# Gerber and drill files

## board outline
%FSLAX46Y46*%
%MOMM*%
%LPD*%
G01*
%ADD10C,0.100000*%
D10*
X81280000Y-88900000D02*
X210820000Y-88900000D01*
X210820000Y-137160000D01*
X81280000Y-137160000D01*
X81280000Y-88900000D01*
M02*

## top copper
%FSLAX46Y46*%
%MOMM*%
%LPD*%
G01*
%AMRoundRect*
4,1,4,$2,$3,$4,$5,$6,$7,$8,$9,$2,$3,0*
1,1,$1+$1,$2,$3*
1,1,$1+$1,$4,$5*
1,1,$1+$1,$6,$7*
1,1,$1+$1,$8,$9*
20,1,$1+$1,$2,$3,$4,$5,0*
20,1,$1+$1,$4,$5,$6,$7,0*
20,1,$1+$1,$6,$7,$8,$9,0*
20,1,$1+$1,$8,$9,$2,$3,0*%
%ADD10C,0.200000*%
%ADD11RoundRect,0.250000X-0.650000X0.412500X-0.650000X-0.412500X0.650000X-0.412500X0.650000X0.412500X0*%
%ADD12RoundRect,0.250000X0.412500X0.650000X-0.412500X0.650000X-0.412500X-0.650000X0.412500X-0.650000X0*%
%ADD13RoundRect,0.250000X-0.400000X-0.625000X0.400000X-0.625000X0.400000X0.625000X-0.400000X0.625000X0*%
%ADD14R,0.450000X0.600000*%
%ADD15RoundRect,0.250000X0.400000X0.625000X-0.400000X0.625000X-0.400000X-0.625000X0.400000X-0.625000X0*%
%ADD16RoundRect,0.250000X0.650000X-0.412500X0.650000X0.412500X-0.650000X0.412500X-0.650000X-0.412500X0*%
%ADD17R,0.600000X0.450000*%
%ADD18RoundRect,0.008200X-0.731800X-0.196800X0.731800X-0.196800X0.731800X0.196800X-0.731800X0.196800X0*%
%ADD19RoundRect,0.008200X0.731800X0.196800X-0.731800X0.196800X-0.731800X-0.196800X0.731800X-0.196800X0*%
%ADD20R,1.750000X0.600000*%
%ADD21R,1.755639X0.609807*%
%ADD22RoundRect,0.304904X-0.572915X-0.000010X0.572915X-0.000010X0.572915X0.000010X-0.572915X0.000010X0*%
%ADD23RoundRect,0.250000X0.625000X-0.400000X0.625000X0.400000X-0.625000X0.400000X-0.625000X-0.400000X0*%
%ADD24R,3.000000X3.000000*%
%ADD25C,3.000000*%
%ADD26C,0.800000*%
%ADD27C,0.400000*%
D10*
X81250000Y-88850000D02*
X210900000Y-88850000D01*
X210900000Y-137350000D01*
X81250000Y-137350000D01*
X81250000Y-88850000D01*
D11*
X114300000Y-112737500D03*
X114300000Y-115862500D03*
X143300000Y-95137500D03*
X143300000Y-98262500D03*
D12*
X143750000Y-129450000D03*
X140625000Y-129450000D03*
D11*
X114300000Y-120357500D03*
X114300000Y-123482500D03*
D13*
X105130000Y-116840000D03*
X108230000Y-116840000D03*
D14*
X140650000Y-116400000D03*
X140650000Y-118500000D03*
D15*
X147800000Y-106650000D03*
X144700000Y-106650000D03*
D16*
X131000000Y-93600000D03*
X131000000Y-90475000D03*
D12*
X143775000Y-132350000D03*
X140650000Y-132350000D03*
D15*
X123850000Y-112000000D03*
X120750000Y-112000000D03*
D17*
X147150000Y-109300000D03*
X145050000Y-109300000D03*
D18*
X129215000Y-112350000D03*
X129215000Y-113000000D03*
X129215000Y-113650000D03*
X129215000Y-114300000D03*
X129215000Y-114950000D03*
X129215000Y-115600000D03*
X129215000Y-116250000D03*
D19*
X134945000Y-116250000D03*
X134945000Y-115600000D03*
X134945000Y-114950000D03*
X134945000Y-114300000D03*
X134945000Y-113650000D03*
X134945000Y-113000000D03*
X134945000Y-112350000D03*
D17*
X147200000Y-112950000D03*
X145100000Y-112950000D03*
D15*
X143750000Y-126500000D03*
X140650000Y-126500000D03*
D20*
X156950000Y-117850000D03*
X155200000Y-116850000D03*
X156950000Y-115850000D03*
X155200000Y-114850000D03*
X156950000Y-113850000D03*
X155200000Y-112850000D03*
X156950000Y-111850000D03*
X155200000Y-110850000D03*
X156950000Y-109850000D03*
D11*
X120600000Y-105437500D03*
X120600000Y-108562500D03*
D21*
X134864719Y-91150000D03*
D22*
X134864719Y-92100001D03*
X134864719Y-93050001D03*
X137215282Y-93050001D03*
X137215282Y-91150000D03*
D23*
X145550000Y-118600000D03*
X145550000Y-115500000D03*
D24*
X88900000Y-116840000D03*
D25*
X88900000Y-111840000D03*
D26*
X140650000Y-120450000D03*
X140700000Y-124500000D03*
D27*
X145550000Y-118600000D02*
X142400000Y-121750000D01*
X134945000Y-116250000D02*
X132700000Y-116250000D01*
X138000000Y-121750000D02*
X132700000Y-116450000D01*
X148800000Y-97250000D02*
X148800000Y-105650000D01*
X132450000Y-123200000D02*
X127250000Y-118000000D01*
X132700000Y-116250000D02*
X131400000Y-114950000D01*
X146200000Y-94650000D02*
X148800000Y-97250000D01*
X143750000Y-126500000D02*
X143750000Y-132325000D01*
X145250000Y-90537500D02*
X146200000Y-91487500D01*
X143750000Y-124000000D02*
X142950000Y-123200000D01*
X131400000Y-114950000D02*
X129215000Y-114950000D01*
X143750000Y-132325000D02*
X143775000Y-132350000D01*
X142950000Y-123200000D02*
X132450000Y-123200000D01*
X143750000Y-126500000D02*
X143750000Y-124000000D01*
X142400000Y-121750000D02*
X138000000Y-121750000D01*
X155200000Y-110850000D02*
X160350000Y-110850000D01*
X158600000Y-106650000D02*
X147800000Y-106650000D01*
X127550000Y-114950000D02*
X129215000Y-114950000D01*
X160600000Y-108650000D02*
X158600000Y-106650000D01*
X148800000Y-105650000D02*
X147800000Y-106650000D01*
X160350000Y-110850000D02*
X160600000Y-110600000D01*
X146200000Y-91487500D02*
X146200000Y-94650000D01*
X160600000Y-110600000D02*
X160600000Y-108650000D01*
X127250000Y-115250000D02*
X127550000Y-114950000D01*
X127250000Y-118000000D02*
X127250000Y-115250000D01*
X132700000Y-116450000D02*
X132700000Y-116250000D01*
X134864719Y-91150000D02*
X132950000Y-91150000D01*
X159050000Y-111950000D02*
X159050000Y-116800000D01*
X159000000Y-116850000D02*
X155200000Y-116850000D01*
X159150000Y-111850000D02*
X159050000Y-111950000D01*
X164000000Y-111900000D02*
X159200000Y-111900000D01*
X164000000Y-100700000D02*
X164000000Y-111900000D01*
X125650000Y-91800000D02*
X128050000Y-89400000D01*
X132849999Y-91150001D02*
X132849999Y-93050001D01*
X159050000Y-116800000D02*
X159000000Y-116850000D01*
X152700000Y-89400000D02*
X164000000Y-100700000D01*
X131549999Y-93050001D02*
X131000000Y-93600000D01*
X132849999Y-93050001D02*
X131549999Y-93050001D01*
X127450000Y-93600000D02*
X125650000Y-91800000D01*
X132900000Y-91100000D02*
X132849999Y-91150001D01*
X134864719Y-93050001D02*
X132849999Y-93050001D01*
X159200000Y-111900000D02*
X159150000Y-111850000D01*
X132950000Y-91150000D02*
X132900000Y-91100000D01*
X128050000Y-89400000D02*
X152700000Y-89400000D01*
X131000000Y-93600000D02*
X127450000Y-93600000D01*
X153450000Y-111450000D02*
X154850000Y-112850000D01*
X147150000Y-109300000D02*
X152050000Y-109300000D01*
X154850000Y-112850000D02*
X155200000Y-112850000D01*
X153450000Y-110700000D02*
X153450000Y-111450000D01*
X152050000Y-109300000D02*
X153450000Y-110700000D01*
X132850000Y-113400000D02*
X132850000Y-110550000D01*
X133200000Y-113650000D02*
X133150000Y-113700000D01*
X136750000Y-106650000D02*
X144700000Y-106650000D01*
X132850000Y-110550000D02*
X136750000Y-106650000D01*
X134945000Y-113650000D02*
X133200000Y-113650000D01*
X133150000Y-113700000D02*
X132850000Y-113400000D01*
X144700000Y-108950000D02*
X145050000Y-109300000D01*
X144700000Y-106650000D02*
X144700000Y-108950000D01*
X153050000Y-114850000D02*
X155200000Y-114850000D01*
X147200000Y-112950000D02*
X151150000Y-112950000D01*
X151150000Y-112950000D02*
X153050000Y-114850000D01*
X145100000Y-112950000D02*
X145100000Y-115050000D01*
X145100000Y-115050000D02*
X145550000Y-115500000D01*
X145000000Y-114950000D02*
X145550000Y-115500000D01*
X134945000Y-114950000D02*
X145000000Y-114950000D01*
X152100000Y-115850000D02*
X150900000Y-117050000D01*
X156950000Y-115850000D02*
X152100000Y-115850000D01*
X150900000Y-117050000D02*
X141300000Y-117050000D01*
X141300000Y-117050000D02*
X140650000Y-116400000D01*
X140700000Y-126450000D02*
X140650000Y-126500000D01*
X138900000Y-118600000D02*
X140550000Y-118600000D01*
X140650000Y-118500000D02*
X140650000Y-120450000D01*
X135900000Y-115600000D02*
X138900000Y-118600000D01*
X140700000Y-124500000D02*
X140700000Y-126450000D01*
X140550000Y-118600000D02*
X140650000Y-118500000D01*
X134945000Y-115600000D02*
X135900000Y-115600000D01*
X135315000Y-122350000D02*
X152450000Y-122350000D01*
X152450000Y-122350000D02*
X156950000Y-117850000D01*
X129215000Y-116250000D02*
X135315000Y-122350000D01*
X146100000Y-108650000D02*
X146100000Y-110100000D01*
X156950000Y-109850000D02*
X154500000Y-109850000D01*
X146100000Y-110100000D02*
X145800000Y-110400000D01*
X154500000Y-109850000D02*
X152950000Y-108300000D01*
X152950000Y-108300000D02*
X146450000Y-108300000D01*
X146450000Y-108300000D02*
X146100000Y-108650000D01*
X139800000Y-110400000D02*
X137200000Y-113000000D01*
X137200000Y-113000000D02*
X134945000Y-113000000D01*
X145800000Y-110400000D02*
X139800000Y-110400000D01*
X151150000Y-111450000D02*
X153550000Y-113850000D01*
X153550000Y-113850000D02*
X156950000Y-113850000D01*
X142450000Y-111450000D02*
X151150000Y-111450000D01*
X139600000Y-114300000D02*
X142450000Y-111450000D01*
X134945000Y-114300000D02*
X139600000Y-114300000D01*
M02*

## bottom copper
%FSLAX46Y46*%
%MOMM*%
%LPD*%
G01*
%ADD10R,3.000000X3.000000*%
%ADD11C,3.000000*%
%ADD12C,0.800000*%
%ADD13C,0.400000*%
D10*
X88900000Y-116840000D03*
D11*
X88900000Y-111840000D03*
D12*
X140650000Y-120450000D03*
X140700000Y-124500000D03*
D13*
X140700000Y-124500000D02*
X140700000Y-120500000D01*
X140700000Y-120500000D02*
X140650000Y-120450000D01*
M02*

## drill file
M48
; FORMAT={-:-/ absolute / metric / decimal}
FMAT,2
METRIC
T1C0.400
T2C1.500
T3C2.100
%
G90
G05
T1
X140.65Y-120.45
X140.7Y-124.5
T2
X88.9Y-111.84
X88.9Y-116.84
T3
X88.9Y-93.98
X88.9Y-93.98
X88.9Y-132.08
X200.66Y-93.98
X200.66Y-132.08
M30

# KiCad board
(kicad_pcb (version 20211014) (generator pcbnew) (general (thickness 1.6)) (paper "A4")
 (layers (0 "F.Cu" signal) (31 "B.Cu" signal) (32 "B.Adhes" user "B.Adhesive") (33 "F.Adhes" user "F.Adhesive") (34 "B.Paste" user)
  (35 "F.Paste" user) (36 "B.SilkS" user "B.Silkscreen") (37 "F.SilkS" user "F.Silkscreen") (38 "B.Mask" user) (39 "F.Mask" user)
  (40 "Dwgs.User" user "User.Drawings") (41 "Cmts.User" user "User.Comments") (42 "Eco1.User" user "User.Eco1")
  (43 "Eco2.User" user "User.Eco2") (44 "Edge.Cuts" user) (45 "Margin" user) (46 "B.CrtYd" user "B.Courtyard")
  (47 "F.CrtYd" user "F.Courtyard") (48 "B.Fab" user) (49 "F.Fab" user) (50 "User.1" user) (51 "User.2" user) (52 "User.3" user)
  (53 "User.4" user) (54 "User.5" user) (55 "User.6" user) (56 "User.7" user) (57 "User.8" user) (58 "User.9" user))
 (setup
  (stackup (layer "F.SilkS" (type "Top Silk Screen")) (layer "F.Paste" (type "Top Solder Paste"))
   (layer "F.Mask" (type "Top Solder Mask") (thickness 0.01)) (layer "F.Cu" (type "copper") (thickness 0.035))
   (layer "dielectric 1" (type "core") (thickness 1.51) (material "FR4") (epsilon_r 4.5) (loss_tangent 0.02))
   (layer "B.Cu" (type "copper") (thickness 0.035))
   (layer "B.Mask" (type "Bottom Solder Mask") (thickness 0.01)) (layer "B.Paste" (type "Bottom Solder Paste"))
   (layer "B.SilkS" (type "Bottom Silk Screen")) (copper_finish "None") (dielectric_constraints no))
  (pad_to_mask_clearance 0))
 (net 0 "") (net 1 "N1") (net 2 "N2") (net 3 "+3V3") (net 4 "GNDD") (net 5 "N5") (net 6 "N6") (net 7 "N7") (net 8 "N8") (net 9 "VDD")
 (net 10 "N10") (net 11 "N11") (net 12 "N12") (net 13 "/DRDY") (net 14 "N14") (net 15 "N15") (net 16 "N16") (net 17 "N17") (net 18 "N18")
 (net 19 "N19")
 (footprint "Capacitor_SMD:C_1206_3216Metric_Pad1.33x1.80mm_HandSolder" (layer "F.Cu") (at 114.3 114.3 -90)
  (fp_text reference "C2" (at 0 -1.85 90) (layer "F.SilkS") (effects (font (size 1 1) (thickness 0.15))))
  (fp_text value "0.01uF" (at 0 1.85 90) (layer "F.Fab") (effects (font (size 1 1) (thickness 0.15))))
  (pad "1" smd roundrect (at -1.5625 0 270) (size 1.325 1.8) (layers "F.Cu" "F.Paste" "F.Mask") (roundrect_rratio 0.188679) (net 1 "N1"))
  (pad "2" smd roundrect (at 1.5625 0 270) (size 1.325 1.8) (layers "F.Cu" "F.Paste" "F.Mask") (roundrect_rratio 0.188679) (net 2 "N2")))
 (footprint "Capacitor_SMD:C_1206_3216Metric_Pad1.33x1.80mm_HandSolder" (layer "F.Cu") (at 143.3 96.7 -90)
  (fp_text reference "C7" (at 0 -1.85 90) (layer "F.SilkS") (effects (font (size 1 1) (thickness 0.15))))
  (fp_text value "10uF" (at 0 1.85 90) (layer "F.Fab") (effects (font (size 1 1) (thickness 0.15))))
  (pad "1" smd roundrect (at -1.5625 0 270) (size 1.325 1.8) (layers "F.Cu" "F.Paste" "F.Mask") (roundrect_rratio 0.188679) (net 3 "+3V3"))
  (pad "2" smd roundrect (at 1.5625 0 270) (size 1.325 1.8) (layers "F.Cu" "F.Paste" "F.Mask") (roundrect_rratio 0.188679) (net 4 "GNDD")))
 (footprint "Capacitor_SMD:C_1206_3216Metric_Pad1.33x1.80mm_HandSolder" (layer "F.Cu") (at 142.1875 129.45 180)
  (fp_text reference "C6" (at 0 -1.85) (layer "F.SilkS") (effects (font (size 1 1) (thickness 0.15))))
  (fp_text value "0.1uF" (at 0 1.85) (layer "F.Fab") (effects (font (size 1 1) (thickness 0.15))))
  (pad "1" smd roundrect (at -1.5625 0 180) (size 1.325 1.8) (layers "F.Cu" "F.Paste" "F.Mask") (roundrect_rratio 0.188679) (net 3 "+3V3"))
  (pad "2" smd roundrect (at 1.5625 0 180) (size 1.325 1.8) (layers "F.Cu" "F.Paste" "F.Mask") (roundrect_rratio 0.188679) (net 4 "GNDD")))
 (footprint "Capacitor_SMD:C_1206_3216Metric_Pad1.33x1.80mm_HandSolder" (layer "F.Cu") (at 114.3 121.92 -90)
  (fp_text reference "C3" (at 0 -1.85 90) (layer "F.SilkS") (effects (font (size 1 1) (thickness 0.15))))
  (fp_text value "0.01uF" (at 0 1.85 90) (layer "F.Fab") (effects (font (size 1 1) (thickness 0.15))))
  (pad "1" smd roundrect (at -1.5625 0 270) (size 1.325 1.8) (layers "F.Cu" "F.Paste" "F.Mask") (roundrect_rratio 0.188679) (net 2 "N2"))
  (pad "2" smd roundrect (at 1.5625 0 270) (size 1.325 1.8) (layers "F.Cu" "F.Paste" "F.Mask") (roundrect_rratio 0.188679) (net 4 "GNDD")))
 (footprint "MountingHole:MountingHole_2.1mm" (layer "F.Cu") (at 200.66 132.08)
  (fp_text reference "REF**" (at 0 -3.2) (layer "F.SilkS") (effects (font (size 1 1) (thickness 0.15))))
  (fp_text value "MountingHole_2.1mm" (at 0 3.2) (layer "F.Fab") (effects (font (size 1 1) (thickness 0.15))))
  (pad "" np_thru_hole circle (at 0 0) (size 2.1 2.1) (drill 2.1) (layers *.Cu *.Mask)))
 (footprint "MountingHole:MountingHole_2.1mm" (layer "F.Cu") (at 88.9 93.98)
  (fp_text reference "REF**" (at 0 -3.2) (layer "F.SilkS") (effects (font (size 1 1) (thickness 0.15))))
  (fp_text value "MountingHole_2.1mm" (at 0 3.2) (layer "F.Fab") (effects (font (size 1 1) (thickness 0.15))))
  (pad "" np_thru_hole circle (at 0 0) (size 2.1 2.1) (drill 2.1) (layers *.Cu *.Mask))
  (pad "" np_thru_hole circle (at 0 0) (size 2.1 2.1) (drill 2.1) (layers *.Cu *.Mask)))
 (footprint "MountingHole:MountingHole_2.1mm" (layer "F.Cu") (at 88.9 132.08)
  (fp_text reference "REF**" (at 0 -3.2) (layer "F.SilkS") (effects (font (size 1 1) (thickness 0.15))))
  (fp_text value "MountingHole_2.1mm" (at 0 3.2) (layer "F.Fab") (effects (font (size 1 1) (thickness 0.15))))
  (pad "" np_thru_hole circle (at 0 0) (size 2.1 2.1) (drill 2.1) (layers *.Cu *.Mask)))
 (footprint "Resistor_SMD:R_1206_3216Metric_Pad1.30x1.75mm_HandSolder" (layer "F.Cu") (at 106.68 116.84)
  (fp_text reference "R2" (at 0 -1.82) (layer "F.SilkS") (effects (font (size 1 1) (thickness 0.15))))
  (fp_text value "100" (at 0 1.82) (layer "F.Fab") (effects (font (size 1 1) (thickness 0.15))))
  (pad "1" smd roundrect (at -1.55 0) (size 1.3 1.75) (layers "F.Cu" "F.Paste" "F.Mask") (roundrect_rratio 0.192308) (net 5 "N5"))
  (pad "2" smd roundrect (at 1.55 0) (size 1.3 1.75) (layers "F.Cu" "F.Paste" "F.Mask") (roundrect_rratio 0.192308) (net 2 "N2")))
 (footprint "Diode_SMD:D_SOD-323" (layer "F.Cu") (at 140.65 117.45 -90)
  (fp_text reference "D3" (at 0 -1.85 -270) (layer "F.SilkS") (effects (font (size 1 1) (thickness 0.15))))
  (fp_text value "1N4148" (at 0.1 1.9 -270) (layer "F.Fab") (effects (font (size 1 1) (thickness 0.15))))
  (pad "1" smd rect (at -1.05 0 270) (size 0.6 0.45) (layers "F.Cu" "F.Paste" "F.Mask") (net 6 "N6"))
  (pad "2" smd rect (at 1.05 0 270) (size 0.6 0.45) (layers "F.Cu" "F.Paste" "F.Mask") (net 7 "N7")))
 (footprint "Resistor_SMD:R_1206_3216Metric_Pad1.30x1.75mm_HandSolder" (layer "F.Cu") (at 146.25 106.65 180)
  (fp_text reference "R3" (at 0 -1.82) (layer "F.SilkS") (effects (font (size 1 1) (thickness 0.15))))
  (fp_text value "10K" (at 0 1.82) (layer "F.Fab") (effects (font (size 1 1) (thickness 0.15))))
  (pad "1" smd roundrect (at -1.55 0 180) (size 1.3 1.75) (layers "F.Cu" "F.Paste" "F.Mask") (roundrect_rratio 0.192308) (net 3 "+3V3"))
  (pad "2" smd roundrect (at 1.55 0 180) (size 1.3 1.75) (layers "F.Cu" "F.Paste" "F.Mask") (roundrect_rratio 0.192308) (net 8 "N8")))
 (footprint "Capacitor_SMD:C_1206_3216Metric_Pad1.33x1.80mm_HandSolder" (layer "F.Cu") (at 131 92.0375 90)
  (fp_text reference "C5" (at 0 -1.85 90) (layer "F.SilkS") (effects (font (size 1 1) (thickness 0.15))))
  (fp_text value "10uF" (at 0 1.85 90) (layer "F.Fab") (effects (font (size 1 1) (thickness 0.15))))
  (pad "1" smd roundrect (at -1.5625 0 90) (size 1.325 1.8) (layers "F.Cu" "F.Paste" "F.Mask") (roundrect_rratio 0.188679) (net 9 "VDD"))
  (pad "2" smd roundrect (at 1.5625 0 90) (size 1.325 1.8) (layers "F.Cu" "F.Paste" "F.Mask") (roundrect_rratio 0.188679) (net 4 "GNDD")))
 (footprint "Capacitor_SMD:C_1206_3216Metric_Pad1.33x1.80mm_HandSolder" (layer "F.Cu") (at 142.2125 132.35 180)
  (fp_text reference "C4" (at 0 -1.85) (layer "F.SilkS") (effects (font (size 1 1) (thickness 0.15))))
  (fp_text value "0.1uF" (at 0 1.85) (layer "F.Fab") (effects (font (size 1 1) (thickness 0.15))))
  (pad "1" smd roundrect (at -1.5625 0 180) (size 1.325 1.8) (layers "F.Cu" "F.Paste" "F.Mask") (roundrect_rratio 0.188679) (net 3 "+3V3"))
  (pad "2" smd roundrect (at 1.5625 0 180) (size 1.325 1.8) (layers "F.Cu" "F.Paste" "F.Mask") (roundrect_rratio 0.188679) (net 4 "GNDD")))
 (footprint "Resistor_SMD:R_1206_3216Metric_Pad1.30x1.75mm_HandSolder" (layer "F.Cu") (at 122.3 112 180)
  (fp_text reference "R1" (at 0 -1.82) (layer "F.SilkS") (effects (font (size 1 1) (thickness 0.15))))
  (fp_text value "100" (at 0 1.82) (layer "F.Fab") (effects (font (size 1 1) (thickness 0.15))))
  (pad "1" smd roundrect (at -1.55 0 180) (size 1.3 1.75) (layers "F.Cu" "F.Paste" "F.Mask") (roundrect_rratio 0.192308) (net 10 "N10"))
  (pad "2" smd roundrect (at 1.55 0 180) (size 1.3 1.75) (layers "F.Cu" "F.Paste" "F.Mask") (roundrect_rratio 0.192308) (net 1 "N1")))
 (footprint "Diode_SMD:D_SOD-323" (layer "F.Cu") (at 146.1 109.3 180)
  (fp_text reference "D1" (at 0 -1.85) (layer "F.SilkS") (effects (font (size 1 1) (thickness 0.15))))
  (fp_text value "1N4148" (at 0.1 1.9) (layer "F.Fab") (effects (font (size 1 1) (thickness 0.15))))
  (pad "1" smd rect (at -1.05 0 180) (size 0.6 0.45) (layers "F.Cu" "F.Paste" "F.Mask") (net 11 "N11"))
  (pad "2" smd rect (at 1.05 0 180) (size 0.6 0.45) (layers "F.Cu" "F.Paste" "F.Mask") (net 8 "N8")))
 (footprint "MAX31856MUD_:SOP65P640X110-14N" (layer "F.Cu") (at 132.08 114.3)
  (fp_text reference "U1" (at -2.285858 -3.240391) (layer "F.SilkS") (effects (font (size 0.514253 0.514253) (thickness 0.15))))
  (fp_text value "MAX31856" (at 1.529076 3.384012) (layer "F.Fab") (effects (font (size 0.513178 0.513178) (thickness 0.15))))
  (pad "1" smd roundrect locked (at -2.865 -1.95) (size 1.48 0.41) (layers "F.Cu" "F.Paste" "F.Mask") (roundrect_rratio 0.02) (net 4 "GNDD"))
  (pad "2" smd roundrect locked (at -2.865 -1.3) (size 1.48 0.41) (layers "F.Cu" "F.Paste" "F.Mask") (roundrect_rratio 0.02) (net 10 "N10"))
  (pad "3" smd roundrect locked (at -2.865 -0.65) (size 1.48 0.41) (layers "F.Cu" "F.Paste" "F.Mask") (roundrect_rratio 0.02) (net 1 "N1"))
  (pad "4" smd roundrect locked (at -2.865 0) (size 1.48 0.41) (layers "F.Cu" "F.Paste") (roundrect_rratio 0.02) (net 2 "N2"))
  (pad "5" smd roundrect locked (at -2.865 0.65) (size 1.48 0.41) (layers "F.Cu" "F.Paste" "F.Mask") (roundrect_rratio 0.02) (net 3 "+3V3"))
  (pad "6" smd roundrect locked (at -2.865 1.3) (size 1.48 0.41) (layers "F.Cu" "F.Paste" "F.Mask") (roundrect_rratio 0.02) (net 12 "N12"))
  (pad "7" smd roundrect locked (at -2.865 1.95) (size 1.48 0.41) (layers "F.Cu" "F.Paste" "F.Mask") (roundrect_rratio 0.02)
   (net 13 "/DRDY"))
  (pad "8" smd roundrect locked (at 2.865 1.95 180) (size 1.48 0.41) (layers "F.Cu" "F.Paste" "F.Mask") (roundrect_rratio 0.02)
   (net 3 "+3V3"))
  (pad "9" smd roundrect locked (at 2.865 1.3 180) (size 1.48 0.41) (layers "F.Cu" "F.Paste" "F.Mask") (roundrect_rratio 0.02) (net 7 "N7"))
  (pad "10" smd roundrect locked (at 2.865 0.65 180) (size 1.48 0.41) (layers "F.Cu" "F.Paste" "F.Mask") (roundrect_rratio 0.02)
   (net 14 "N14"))
  (pad "11" smd roundrect locked (at 2.865 0 180) (size 1.48 0.41) (layers "F.Cu" "F.Paste" "F.Mask") (roundrect_rratio 0.02) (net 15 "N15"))
  (pad "12" smd roundrect locked (at 2.865 -0.65 180) (size 1.48 0.41) (layers "F.Cu" "F.Paste" "F.Mask") (roundrect_rratio 0.02)
   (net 8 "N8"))
  (pad "13" smd roundrect locked (at 2.865 -1.3 180) (size 1.48 0.41) (layers "F.Cu" "F.Paste" "F.Mask") (roundrect_rratio 0.02)
   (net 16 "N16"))
  (pad "14" smd roundrect locked (at 2.865 -1.95 180) (size 1.48 0.41) (layers "F.Cu" "F.Paste" "F.Mask") (roundrect_rratio 0.02)
   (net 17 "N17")))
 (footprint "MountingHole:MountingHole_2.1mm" (layer "F.Cu") (at 200.66 93.98)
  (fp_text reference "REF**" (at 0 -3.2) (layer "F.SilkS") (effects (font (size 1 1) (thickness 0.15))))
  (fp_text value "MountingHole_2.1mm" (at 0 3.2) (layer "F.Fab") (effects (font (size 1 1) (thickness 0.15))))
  (pad "" np_thru_hole circle (at 0 0) (size 2.1 2.1) (drill 2.1) (layers *.Cu *.Mask)))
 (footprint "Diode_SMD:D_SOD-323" (layer "F.Cu") (at 146.15 112.95 180)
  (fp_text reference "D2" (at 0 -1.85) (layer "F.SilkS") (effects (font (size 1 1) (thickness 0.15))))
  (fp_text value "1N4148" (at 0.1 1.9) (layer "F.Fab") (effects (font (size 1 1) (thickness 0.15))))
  (pad "1" smd rect (at -1.05 0 180) (size 0.6 0.45) (layers "F.Cu" "F.Paste" "F.Mask") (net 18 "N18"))
  (pad "2" smd rect (at 1.05 0 180) (size 0.6 0.45) (layers "F.Cu" "F.Paste" "F.Mask") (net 14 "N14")))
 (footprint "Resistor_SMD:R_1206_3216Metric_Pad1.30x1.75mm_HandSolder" (layer "F.Cu") (at 142.2 126.5 180)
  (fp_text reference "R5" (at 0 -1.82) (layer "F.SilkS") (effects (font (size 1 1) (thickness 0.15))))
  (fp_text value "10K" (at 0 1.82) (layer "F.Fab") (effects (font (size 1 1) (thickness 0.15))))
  (pad "1" smd roundrect (at -1.55 0 180) (size 1.3 1.75) (layers "F.Cu" "F.Paste" "F.Mask") (roundrect_rratio 0.192308) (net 3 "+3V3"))
  (pad "2" smd roundrect (at 1.55 0 180) (size 1.3 1.75) (layers "F.Cu" "F.Paste" "F.Mask") (roundrect_rratio 0.192308) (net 7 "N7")))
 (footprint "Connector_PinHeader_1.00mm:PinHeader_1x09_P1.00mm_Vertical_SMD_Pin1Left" (layer "F.Cu") (at 156.075 113.85 180)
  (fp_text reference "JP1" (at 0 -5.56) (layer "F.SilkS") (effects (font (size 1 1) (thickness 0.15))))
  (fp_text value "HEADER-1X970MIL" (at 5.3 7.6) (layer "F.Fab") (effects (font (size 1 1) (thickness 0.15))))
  (pad "1" smd rect (at -0.875 -4 180) (size 1.75 0.6) (layers "F.Cu" "F.Paste" "F.Mask") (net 13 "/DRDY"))
  (pad "2" smd rect (at 0.875 -3 180) (size 1.75 0.6) (layers "F.Cu" "F.Paste" "F.Mask") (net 9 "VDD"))
  (pad "3" smd rect (at -0.875 -2 180) (size 1.75 0.6) (layers "F.Cu" "F.Paste" "F.Mask") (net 6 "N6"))
  (pad "4" smd rect (at 0.875 -1 180) (size 1.75 0.6) (layers "F.Cu" "F.Paste" "F.Mask") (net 18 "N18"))
  (pad "5" smd rect (at -0.875 0 180) (size 1.75 0.6) (layers "F.Cu" "F.Paste" "F.Mask") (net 15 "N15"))
  (pad "6" smd rect (at 0.875 1 180) (size 1.75 0.6) (layers "F.Cu" "F.Paste" "F.Mask") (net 11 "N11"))
  (pad "7" smd rect (at -0.875 2 180) (size 1.75 0.6) (layers "F.Cu" "F.Paste" "F.Mask") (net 4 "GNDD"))
  (pad "8" smd rect (at 0.875 3 180) (size 1.75 0.6) (layers "F.Cu" "F.Paste" "F.Mask") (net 3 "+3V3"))
  (pad "9" smd rect (at -0.875 4 180) (size 1.75 0.6) (layers "F.Cu" "F.Paste" "F.Mask") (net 16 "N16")))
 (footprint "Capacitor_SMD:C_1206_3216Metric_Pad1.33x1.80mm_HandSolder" (layer "F.Cu") (at 120.6 107 -90)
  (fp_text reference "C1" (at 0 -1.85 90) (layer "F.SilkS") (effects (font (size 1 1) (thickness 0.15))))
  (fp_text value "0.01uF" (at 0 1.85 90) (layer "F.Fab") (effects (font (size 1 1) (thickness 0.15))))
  (pad "1" smd roundrect (at -1.5625 0 270) (size 1.325 1.8) (layers "F.Cu" "F.Paste" "F.Mask") (roundrect_rratio 0.188679) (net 4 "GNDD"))
  (pad "2" smd roundrect (at 1.5625 0 270) (size 1.325 1.8) (layers "F.Cu" "F.Paste" "F.Mask") (roundrect_rratio 0.188679) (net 1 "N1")))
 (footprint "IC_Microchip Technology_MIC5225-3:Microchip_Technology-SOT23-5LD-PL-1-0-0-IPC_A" (layer "F.Cu") (at 136.04 92.1)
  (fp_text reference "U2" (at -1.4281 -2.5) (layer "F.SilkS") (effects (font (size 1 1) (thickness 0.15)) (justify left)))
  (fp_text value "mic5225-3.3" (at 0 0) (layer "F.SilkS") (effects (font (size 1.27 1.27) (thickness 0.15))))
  (pad "1" smd rect locked (at -1.175281 -0.95) (size 1.755639 0.609807) (layers "F.Cu" "F.Paste" "F.Mask") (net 9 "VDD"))
  (pad "2" smd roundrect locked (at -1.175281 0.000001) (size 1.755639 0.609807) (layers "F.Cu" "F.Paste" "F.Mask") (roundrect_rratio 0.5)
   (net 4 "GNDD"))
  (pad "3" smd roundrect locked (at -1.175281 0.950001) (size 1.755639 0.609807) (layers "F.Cu" "F.Paste" "F.Mask") (roundrect_rratio 0.5)
   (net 9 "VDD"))
  (pad "4" smd roundrect locked (at 1.175282 0.950001) (size 1.755639 0.609807) (layers "F.Cu" "F.Paste" "F.Mask") (roundrect_rratio 0.5)
   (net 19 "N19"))
  (pad "5" smd roundrect locked (at 1.175282 -0.95) (size 1.755639 0.609807) (layers "F.Cu" "F.Paste" "F.Mask") (roundrect_rratio 0.5)
   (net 3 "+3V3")))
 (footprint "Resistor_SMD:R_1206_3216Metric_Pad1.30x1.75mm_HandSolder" (layer "F.Cu") (at 145.55 117.05 90)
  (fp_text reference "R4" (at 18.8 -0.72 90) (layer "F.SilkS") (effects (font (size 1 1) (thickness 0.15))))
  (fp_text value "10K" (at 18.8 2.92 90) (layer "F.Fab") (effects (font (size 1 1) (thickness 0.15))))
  (pad "1" smd roundrect (at -1.55 0 90) (size 1.3 1.75) (layers "F.Cu" "F.Paste" "F.Mask") (roundrect_rratio 0.192308) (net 3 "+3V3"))
  (pad "2" smd roundrect (at 1.55 0 90) (size 1.3 1.75) (layers "F.Cu" "F.Paste" "F.Mask") (roundrect_rratio 0.192308) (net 14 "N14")))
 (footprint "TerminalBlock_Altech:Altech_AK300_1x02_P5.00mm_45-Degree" (layer "B.Cu") (at 88.9 116.84 90)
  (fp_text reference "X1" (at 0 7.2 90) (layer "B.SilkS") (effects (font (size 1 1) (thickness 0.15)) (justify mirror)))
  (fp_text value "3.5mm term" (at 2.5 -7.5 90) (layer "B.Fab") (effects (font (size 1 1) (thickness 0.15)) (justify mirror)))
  (pad "1" thru_hole rect (at 0 0 90) (size 3 3) (drill 1.5) (layers *.Cu *.Mask) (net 5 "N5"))
  (pad "2" thru_hole circle (at 5 0 90) (size 3 3) (drill 1.5) (layers *.Cu *.Mask) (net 10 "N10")))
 (gr_rect (start 81.25 137.35) (end 210.9 88.85) (layer "F.Cu") (width 0.2) (fill none))
 (gr_rect (start 210.82 137.16) (end 81.28 88.9) (layer "Edge.Cuts") (width 0.1) (fill none))
 (via (at 140.65 120.45) (size 0.8) (drill 0.4) (layers "F.Cu" "B.Cu") (free) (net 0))
 (segment (start 145.55 118.6) (end 142.4 121.75) (width 0.4) (layer "F.Cu") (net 3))
 (segment (start 134.945 116.25) (end 132.7 116.25) (width 0.4) (layer "F.Cu") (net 3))
 (segment (start 138 121.75) (end 132.7 116.45) (width 0.4) (layer "F.Cu") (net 3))
 (segment (start 148.8 97.25) (end 148.8 105.65) (width 0.4) (layer "F.Cu") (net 3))
 (segment (start 132.45 123.2) (end 127.25 118) (width 0.4) (layer "F.Cu") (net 3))
 (segment (start 132.7 116.25) (end 131.4 114.95) (width 0.4) (layer "F.Cu") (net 3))
 (segment (start 146.2 94.65) (end 148.8 97.25) (width 0.4) (layer "F.Cu") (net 3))
 (segment (start 143.75 126.5) (end 143.75 132.325) (width 0.4) (layer "F.Cu") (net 3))
 (segment (start 145.25 90.5375) (end 146.2 91.4875) (width 0.4) (layer "F.Cu") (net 3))
 (segment (start 143.75 124) (end 142.95 123.2) (width 0.4) (layer "F.Cu") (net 3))
 (segment (start 131.4 114.95) (end 129.215 114.95) (width 0.4) (layer "F.Cu") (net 3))
 (segment (start 143.75 132.325) (end 143.775 132.35) (width 0.4) (layer "F.Cu") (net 3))
 (segment (start 142.95 123.2) (end 132.45 123.2) (width 0.4) (layer "F.Cu") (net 3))
 (segment (start 143.75 126.5) (end 143.75 124) (width 0.4) (layer "F.Cu") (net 3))
 (segment (start 142.4 121.75) (end 138 121.75) (width 0.4) (layer "F.Cu") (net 3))
 (segment (start 155.2 110.85) (end 160.35 110.85) (width 0.4) (layer "F.Cu") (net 3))
 (segment (start 158.6 106.65) (end 147.8 106.65) (width 0.4) (layer "F.Cu") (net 3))
 (segment (start 127.55 114.95) (end 129.215 114.95) (width 0.4) (layer "F.Cu") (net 3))
 (segment (start 160.6 108.65) (end 158.6 106.65) (width 0.4) (layer "F.Cu") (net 3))
 (segment (start 148.8 105.65) (end 147.8 106.65) (width 0.4) (layer "F.Cu") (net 3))
 (segment (start 160.35 110.85) (end 160.6 110.6) (width 0.4) (layer "F.Cu") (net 3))
 (segment (start 146.2 91.4875) (end 146.2 94.65) (width 0.4) (layer "F.Cu") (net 3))
 (segment (start 160.6 110.6) (end 160.6 108.65) (width 0.4) (layer "F.Cu") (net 3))
 (segment (start 127.25 115.25) (end 127.55 114.95) (width 0.4) (layer "F.Cu") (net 3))
 (segment (start 127.25 118) (end 127.25 115.25) (width 0.4) (layer "F.Cu") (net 3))
 (segment (start 132.7 116.45) (end 132.7 116.25) (width 0.4) (layer "F.Cu") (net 3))
 (segment (start 134.864719 91.15) (end 132.95 91.15) (width 0.4) (layer "F.Cu") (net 9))
 (segment (start 159.05 111.95) (end 159.05 116.8) (width 0.4) (layer "F.Cu") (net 9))
 (segment (start 159 116.85) (end 155.2 116.85) (width 0.4) (layer "F.Cu") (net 9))
 (segment (start 159.15 111.85) (end 159.05 111.95) (width 0.4) (layer "F.Cu") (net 9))
 (segment (start 164 111.9) (end 159.2 111.9) (width 0.4) (layer "F.Cu") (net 9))
 (segment (start 164 100.7) (end 164 111.9) (width 0.4) (layer "F.Cu") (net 9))
 (segment (start 125.65 91.8) (end 128.05 89.4) (width 0.4) (layer "F.Cu") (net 9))
 (segment (start 132.849999 91.150001) (end 132.849999 93.050001) (width 0.4) (layer "F.Cu") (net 9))
 (segment (start 159.05 116.8) (end 159 116.85) (width 0.4) (layer "F.Cu") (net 9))
 (segment (start 152.7 89.4) (end 164 100.7) (width 0.4) (layer "F.Cu") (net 9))
 (segment (start 131.549999 93.050001) (end 131 93.6) (width 0.4) (layer "F.Cu") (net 9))
 (segment (start 132.849999 93.050001) (end 131.549999 93.050001) (width 0.4) (layer "F.Cu") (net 9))
 (segment (start 127.45 93.6) (end 125.65 91.8) (width 0.4) (layer "F.Cu") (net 9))
 (segment (start 132.9 91.1) (end 132.849999 91.150001) (width 0.4) (layer "F.Cu") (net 9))
 (segment (start 134.864719 93.050001) (end 132.849999 93.050001) (width 0.4) (layer "F.Cu") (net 9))
 (segment (start 159.2 111.9) (end 159.15 111.85) (width 0.4) (layer "F.Cu") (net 9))
 (segment (start 132.95 91.15) (end 132.9 91.1) (width 0.4) (layer "F.Cu") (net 9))
 (segment (start 128.05 89.4) (end 152.7 89.4) (width 0.4) (layer "F.Cu") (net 9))
 (segment (start 131 93.6) (end 127.45 93.6) (width 0.4) (layer "F.Cu") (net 9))
 (segment (start 153.45 111.45) (end 154.85 112.85) (width 0.4) (layer "F.Cu") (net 11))
 (segment (start 147.15 109.3) (end 152.05 109.3) (width 0.4) (layer "F.Cu") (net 11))
 (segment (start 154.85 112.85) (end 155.2 112.85) (width 0.4) (layer "F.Cu") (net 11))
 (segment (start 153.45 110.7) (end 153.45 111.45) (width 0.4) (layer "F.Cu") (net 11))
 (segment (start 152.05 109.3) (end 153.45 110.7) (width 0.4) (layer "F.Cu") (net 11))
 (segment (start 132.85 113.4) (end 132.85 110.55) (width 0.4) (layer "F.Cu") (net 8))
 (segment (start 133.2 113.65) (end 133.15 113.7) (width 0.4) (layer "F.Cu") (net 8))
 (segment (start 136.75 106.65) (end 144.7 106.65) (width 0.4) (layer "F.Cu") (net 8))
 (segment (start 132.85 110.55) (end 136.75 106.65) (width 0.4) (layer "F.Cu") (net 8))
 (segment (start 134.945 113.65) (end 133.2 113.65) (width 0.4) (layer "F.Cu") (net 8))
 (segment (start 133.15 113.7) (end 132.85 113.4) (width 0.4) (layer "F.Cu") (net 8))
 (segment (start 144.7 108.95) (end 145.05 109.3) (width 0.4) (layer "F.Cu") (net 8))
 (segment (start 144.7 106.65) (end 144.7 108.95) (width 0.4) (layer "F.Cu") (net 8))
 (segment (start 153.05 114.85) (end 155.2 114.85) (width 0.4) (layer "F.Cu") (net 18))
 (segment (start 147.2 112.95) (end 151.15 112.95) (width 0.4) (layer "F.Cu") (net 18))
 (segment (start 151.15 112.95) (end 153.05 114.85) (width 0.4) (layer "F.Cu") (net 18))
 (segment (start 145.1 112.95) (end 145.1 115.05) (width 0.4) (layer "F.Cu") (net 14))
 (segment (start 145.1 115.05) (end 145.55 115.5) (width 0.4) (layer "F.Cu") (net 14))
 (segment (start 145 114.95) (end 145.55 115.5) (width 0.4) (layer "F.Cu") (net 14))
 (segment (start 134.945 114.95) (end 145 114.95) (width 0.4) (layer "F.Cu") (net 14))
 (segment (start 152.1 115.85) (end 150.9 117.05) (width 0.4) (layer "F.Cu") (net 6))
 (segment (start 156.95 115.85) (end 152.1 115.85) (width 0.4) (layer "F.Cu") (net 6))
 (segment (start 150.9 117.05) (end 141.3 117.05) (width 0.4) (layer "F.Cu") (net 6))
 (segment (start 141.3 117.05) (end 140.65 116.4) (width 0.4) (layer "F.Cu") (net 6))
 (segment (start 140.7 126.45) (end 140.65 126.5) (width 0.4) (layer "F.Cu") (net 7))
 (segment (start 138.9 118.6) (end 140.55 118.6) (width 0.4) (layer "F.Cu") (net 7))
 (segment (start 140.65 118.5) (end 140.65 120.45) (width 0.4) (layer "F.Cu") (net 7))
 (segment (start 135.9 115.6) (end 138.9 118.6) (width 0.4) (layer "F.Cu") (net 7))
 (segment (start 140.7 124.5) (end 140.7 126.45) (width 0.4) (layer "F.Cu") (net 7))
 (segment (start 140.55 118.6) (end 140.65 118.5) (width 0.4) (layer "F.Cu") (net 7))
 (segment (start 134.945 115.6) (end 135.9 115.6) (width 0.4) (layer "F.Cu") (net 7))
 (via (at 140.7 124.5) (size 0.8) (drill 0.4) (layers "F.Cu" "B.Cu") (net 7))
 (segment (start 140.7 124.5) (end 140.7 120.5) (width 0.4) (layer "B.Cu") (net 7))
 (segment (start 140.7 120.5) (end 140.65 120.45) (width 0.4) (layer "B.Cu") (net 7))
 (segment (start 135.315 122.35) (end 152.45 122.35) (width 0.4) (layer "F.Cu") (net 13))
 (segment (start 152.45 122.35) (end 156.95 117.85) (width 0.4) (layer "F.Cu") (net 13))
 (segment (start 129.215 116.25) (end 135.315 122.35) (width 0.4) (layer "F.Cu") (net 13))
 (segment (start 146.1 108.65) (end 146.1 110.1) (width 0.4) (layer "F.Cu") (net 16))
 (segment (start 156.95 109.85) (end 154.5 109.85) (width 0.4) (layer "F.Cu") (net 16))
 (segment (start 146.1 110.1) (end 145.8 110.4) (width 0.4) (layer "F.Cu") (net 16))
 (segment (start 154.5 109.85) (end 152.95 108.3) (width 0.4) (layer "F.Cu") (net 16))
 (segment (start 152.95 108.3) (end 146.45 108.3) (width 0.4) (layer "F.Cu") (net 16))
 (segment (start 146.45 108.3) (end 146.1 108.65) (width 0.4) (layer "F.Cu") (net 16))
 (segment (start 139.8 110.4) (end 137.2 113) (width 0.4) (layer "F.Cu") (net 16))
 (segment (start 137.2 113) (end 134.945 113) (width 0.4) (layer "F.Cu") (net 16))
 (segment (start 145.8 110.4) (end 139.8 110.4) (width 0.4) (layer "F.Cu") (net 16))
 (segment (start 151.15 111.45) (end 153.55 113.85) (width 0.4) (layer "F.Cu") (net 15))
 (segment (start 153.55 113.85) (end 156.95 113.85) (width 0.4) (layer "F.Cu") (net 15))
 (segment (start 142.45 111.45) (end 151.15 111.45) (width 0.4) (layer "F.Cu") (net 15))
 (segment (start 139.6 114.3) (end 142.45 111.45) (width 0.4) (layer "F.Cu") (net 15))
 (segment (start 134.945 114.3) (end 139.6 114.3) (width 0.4) (layer "F.Cu") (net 15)))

